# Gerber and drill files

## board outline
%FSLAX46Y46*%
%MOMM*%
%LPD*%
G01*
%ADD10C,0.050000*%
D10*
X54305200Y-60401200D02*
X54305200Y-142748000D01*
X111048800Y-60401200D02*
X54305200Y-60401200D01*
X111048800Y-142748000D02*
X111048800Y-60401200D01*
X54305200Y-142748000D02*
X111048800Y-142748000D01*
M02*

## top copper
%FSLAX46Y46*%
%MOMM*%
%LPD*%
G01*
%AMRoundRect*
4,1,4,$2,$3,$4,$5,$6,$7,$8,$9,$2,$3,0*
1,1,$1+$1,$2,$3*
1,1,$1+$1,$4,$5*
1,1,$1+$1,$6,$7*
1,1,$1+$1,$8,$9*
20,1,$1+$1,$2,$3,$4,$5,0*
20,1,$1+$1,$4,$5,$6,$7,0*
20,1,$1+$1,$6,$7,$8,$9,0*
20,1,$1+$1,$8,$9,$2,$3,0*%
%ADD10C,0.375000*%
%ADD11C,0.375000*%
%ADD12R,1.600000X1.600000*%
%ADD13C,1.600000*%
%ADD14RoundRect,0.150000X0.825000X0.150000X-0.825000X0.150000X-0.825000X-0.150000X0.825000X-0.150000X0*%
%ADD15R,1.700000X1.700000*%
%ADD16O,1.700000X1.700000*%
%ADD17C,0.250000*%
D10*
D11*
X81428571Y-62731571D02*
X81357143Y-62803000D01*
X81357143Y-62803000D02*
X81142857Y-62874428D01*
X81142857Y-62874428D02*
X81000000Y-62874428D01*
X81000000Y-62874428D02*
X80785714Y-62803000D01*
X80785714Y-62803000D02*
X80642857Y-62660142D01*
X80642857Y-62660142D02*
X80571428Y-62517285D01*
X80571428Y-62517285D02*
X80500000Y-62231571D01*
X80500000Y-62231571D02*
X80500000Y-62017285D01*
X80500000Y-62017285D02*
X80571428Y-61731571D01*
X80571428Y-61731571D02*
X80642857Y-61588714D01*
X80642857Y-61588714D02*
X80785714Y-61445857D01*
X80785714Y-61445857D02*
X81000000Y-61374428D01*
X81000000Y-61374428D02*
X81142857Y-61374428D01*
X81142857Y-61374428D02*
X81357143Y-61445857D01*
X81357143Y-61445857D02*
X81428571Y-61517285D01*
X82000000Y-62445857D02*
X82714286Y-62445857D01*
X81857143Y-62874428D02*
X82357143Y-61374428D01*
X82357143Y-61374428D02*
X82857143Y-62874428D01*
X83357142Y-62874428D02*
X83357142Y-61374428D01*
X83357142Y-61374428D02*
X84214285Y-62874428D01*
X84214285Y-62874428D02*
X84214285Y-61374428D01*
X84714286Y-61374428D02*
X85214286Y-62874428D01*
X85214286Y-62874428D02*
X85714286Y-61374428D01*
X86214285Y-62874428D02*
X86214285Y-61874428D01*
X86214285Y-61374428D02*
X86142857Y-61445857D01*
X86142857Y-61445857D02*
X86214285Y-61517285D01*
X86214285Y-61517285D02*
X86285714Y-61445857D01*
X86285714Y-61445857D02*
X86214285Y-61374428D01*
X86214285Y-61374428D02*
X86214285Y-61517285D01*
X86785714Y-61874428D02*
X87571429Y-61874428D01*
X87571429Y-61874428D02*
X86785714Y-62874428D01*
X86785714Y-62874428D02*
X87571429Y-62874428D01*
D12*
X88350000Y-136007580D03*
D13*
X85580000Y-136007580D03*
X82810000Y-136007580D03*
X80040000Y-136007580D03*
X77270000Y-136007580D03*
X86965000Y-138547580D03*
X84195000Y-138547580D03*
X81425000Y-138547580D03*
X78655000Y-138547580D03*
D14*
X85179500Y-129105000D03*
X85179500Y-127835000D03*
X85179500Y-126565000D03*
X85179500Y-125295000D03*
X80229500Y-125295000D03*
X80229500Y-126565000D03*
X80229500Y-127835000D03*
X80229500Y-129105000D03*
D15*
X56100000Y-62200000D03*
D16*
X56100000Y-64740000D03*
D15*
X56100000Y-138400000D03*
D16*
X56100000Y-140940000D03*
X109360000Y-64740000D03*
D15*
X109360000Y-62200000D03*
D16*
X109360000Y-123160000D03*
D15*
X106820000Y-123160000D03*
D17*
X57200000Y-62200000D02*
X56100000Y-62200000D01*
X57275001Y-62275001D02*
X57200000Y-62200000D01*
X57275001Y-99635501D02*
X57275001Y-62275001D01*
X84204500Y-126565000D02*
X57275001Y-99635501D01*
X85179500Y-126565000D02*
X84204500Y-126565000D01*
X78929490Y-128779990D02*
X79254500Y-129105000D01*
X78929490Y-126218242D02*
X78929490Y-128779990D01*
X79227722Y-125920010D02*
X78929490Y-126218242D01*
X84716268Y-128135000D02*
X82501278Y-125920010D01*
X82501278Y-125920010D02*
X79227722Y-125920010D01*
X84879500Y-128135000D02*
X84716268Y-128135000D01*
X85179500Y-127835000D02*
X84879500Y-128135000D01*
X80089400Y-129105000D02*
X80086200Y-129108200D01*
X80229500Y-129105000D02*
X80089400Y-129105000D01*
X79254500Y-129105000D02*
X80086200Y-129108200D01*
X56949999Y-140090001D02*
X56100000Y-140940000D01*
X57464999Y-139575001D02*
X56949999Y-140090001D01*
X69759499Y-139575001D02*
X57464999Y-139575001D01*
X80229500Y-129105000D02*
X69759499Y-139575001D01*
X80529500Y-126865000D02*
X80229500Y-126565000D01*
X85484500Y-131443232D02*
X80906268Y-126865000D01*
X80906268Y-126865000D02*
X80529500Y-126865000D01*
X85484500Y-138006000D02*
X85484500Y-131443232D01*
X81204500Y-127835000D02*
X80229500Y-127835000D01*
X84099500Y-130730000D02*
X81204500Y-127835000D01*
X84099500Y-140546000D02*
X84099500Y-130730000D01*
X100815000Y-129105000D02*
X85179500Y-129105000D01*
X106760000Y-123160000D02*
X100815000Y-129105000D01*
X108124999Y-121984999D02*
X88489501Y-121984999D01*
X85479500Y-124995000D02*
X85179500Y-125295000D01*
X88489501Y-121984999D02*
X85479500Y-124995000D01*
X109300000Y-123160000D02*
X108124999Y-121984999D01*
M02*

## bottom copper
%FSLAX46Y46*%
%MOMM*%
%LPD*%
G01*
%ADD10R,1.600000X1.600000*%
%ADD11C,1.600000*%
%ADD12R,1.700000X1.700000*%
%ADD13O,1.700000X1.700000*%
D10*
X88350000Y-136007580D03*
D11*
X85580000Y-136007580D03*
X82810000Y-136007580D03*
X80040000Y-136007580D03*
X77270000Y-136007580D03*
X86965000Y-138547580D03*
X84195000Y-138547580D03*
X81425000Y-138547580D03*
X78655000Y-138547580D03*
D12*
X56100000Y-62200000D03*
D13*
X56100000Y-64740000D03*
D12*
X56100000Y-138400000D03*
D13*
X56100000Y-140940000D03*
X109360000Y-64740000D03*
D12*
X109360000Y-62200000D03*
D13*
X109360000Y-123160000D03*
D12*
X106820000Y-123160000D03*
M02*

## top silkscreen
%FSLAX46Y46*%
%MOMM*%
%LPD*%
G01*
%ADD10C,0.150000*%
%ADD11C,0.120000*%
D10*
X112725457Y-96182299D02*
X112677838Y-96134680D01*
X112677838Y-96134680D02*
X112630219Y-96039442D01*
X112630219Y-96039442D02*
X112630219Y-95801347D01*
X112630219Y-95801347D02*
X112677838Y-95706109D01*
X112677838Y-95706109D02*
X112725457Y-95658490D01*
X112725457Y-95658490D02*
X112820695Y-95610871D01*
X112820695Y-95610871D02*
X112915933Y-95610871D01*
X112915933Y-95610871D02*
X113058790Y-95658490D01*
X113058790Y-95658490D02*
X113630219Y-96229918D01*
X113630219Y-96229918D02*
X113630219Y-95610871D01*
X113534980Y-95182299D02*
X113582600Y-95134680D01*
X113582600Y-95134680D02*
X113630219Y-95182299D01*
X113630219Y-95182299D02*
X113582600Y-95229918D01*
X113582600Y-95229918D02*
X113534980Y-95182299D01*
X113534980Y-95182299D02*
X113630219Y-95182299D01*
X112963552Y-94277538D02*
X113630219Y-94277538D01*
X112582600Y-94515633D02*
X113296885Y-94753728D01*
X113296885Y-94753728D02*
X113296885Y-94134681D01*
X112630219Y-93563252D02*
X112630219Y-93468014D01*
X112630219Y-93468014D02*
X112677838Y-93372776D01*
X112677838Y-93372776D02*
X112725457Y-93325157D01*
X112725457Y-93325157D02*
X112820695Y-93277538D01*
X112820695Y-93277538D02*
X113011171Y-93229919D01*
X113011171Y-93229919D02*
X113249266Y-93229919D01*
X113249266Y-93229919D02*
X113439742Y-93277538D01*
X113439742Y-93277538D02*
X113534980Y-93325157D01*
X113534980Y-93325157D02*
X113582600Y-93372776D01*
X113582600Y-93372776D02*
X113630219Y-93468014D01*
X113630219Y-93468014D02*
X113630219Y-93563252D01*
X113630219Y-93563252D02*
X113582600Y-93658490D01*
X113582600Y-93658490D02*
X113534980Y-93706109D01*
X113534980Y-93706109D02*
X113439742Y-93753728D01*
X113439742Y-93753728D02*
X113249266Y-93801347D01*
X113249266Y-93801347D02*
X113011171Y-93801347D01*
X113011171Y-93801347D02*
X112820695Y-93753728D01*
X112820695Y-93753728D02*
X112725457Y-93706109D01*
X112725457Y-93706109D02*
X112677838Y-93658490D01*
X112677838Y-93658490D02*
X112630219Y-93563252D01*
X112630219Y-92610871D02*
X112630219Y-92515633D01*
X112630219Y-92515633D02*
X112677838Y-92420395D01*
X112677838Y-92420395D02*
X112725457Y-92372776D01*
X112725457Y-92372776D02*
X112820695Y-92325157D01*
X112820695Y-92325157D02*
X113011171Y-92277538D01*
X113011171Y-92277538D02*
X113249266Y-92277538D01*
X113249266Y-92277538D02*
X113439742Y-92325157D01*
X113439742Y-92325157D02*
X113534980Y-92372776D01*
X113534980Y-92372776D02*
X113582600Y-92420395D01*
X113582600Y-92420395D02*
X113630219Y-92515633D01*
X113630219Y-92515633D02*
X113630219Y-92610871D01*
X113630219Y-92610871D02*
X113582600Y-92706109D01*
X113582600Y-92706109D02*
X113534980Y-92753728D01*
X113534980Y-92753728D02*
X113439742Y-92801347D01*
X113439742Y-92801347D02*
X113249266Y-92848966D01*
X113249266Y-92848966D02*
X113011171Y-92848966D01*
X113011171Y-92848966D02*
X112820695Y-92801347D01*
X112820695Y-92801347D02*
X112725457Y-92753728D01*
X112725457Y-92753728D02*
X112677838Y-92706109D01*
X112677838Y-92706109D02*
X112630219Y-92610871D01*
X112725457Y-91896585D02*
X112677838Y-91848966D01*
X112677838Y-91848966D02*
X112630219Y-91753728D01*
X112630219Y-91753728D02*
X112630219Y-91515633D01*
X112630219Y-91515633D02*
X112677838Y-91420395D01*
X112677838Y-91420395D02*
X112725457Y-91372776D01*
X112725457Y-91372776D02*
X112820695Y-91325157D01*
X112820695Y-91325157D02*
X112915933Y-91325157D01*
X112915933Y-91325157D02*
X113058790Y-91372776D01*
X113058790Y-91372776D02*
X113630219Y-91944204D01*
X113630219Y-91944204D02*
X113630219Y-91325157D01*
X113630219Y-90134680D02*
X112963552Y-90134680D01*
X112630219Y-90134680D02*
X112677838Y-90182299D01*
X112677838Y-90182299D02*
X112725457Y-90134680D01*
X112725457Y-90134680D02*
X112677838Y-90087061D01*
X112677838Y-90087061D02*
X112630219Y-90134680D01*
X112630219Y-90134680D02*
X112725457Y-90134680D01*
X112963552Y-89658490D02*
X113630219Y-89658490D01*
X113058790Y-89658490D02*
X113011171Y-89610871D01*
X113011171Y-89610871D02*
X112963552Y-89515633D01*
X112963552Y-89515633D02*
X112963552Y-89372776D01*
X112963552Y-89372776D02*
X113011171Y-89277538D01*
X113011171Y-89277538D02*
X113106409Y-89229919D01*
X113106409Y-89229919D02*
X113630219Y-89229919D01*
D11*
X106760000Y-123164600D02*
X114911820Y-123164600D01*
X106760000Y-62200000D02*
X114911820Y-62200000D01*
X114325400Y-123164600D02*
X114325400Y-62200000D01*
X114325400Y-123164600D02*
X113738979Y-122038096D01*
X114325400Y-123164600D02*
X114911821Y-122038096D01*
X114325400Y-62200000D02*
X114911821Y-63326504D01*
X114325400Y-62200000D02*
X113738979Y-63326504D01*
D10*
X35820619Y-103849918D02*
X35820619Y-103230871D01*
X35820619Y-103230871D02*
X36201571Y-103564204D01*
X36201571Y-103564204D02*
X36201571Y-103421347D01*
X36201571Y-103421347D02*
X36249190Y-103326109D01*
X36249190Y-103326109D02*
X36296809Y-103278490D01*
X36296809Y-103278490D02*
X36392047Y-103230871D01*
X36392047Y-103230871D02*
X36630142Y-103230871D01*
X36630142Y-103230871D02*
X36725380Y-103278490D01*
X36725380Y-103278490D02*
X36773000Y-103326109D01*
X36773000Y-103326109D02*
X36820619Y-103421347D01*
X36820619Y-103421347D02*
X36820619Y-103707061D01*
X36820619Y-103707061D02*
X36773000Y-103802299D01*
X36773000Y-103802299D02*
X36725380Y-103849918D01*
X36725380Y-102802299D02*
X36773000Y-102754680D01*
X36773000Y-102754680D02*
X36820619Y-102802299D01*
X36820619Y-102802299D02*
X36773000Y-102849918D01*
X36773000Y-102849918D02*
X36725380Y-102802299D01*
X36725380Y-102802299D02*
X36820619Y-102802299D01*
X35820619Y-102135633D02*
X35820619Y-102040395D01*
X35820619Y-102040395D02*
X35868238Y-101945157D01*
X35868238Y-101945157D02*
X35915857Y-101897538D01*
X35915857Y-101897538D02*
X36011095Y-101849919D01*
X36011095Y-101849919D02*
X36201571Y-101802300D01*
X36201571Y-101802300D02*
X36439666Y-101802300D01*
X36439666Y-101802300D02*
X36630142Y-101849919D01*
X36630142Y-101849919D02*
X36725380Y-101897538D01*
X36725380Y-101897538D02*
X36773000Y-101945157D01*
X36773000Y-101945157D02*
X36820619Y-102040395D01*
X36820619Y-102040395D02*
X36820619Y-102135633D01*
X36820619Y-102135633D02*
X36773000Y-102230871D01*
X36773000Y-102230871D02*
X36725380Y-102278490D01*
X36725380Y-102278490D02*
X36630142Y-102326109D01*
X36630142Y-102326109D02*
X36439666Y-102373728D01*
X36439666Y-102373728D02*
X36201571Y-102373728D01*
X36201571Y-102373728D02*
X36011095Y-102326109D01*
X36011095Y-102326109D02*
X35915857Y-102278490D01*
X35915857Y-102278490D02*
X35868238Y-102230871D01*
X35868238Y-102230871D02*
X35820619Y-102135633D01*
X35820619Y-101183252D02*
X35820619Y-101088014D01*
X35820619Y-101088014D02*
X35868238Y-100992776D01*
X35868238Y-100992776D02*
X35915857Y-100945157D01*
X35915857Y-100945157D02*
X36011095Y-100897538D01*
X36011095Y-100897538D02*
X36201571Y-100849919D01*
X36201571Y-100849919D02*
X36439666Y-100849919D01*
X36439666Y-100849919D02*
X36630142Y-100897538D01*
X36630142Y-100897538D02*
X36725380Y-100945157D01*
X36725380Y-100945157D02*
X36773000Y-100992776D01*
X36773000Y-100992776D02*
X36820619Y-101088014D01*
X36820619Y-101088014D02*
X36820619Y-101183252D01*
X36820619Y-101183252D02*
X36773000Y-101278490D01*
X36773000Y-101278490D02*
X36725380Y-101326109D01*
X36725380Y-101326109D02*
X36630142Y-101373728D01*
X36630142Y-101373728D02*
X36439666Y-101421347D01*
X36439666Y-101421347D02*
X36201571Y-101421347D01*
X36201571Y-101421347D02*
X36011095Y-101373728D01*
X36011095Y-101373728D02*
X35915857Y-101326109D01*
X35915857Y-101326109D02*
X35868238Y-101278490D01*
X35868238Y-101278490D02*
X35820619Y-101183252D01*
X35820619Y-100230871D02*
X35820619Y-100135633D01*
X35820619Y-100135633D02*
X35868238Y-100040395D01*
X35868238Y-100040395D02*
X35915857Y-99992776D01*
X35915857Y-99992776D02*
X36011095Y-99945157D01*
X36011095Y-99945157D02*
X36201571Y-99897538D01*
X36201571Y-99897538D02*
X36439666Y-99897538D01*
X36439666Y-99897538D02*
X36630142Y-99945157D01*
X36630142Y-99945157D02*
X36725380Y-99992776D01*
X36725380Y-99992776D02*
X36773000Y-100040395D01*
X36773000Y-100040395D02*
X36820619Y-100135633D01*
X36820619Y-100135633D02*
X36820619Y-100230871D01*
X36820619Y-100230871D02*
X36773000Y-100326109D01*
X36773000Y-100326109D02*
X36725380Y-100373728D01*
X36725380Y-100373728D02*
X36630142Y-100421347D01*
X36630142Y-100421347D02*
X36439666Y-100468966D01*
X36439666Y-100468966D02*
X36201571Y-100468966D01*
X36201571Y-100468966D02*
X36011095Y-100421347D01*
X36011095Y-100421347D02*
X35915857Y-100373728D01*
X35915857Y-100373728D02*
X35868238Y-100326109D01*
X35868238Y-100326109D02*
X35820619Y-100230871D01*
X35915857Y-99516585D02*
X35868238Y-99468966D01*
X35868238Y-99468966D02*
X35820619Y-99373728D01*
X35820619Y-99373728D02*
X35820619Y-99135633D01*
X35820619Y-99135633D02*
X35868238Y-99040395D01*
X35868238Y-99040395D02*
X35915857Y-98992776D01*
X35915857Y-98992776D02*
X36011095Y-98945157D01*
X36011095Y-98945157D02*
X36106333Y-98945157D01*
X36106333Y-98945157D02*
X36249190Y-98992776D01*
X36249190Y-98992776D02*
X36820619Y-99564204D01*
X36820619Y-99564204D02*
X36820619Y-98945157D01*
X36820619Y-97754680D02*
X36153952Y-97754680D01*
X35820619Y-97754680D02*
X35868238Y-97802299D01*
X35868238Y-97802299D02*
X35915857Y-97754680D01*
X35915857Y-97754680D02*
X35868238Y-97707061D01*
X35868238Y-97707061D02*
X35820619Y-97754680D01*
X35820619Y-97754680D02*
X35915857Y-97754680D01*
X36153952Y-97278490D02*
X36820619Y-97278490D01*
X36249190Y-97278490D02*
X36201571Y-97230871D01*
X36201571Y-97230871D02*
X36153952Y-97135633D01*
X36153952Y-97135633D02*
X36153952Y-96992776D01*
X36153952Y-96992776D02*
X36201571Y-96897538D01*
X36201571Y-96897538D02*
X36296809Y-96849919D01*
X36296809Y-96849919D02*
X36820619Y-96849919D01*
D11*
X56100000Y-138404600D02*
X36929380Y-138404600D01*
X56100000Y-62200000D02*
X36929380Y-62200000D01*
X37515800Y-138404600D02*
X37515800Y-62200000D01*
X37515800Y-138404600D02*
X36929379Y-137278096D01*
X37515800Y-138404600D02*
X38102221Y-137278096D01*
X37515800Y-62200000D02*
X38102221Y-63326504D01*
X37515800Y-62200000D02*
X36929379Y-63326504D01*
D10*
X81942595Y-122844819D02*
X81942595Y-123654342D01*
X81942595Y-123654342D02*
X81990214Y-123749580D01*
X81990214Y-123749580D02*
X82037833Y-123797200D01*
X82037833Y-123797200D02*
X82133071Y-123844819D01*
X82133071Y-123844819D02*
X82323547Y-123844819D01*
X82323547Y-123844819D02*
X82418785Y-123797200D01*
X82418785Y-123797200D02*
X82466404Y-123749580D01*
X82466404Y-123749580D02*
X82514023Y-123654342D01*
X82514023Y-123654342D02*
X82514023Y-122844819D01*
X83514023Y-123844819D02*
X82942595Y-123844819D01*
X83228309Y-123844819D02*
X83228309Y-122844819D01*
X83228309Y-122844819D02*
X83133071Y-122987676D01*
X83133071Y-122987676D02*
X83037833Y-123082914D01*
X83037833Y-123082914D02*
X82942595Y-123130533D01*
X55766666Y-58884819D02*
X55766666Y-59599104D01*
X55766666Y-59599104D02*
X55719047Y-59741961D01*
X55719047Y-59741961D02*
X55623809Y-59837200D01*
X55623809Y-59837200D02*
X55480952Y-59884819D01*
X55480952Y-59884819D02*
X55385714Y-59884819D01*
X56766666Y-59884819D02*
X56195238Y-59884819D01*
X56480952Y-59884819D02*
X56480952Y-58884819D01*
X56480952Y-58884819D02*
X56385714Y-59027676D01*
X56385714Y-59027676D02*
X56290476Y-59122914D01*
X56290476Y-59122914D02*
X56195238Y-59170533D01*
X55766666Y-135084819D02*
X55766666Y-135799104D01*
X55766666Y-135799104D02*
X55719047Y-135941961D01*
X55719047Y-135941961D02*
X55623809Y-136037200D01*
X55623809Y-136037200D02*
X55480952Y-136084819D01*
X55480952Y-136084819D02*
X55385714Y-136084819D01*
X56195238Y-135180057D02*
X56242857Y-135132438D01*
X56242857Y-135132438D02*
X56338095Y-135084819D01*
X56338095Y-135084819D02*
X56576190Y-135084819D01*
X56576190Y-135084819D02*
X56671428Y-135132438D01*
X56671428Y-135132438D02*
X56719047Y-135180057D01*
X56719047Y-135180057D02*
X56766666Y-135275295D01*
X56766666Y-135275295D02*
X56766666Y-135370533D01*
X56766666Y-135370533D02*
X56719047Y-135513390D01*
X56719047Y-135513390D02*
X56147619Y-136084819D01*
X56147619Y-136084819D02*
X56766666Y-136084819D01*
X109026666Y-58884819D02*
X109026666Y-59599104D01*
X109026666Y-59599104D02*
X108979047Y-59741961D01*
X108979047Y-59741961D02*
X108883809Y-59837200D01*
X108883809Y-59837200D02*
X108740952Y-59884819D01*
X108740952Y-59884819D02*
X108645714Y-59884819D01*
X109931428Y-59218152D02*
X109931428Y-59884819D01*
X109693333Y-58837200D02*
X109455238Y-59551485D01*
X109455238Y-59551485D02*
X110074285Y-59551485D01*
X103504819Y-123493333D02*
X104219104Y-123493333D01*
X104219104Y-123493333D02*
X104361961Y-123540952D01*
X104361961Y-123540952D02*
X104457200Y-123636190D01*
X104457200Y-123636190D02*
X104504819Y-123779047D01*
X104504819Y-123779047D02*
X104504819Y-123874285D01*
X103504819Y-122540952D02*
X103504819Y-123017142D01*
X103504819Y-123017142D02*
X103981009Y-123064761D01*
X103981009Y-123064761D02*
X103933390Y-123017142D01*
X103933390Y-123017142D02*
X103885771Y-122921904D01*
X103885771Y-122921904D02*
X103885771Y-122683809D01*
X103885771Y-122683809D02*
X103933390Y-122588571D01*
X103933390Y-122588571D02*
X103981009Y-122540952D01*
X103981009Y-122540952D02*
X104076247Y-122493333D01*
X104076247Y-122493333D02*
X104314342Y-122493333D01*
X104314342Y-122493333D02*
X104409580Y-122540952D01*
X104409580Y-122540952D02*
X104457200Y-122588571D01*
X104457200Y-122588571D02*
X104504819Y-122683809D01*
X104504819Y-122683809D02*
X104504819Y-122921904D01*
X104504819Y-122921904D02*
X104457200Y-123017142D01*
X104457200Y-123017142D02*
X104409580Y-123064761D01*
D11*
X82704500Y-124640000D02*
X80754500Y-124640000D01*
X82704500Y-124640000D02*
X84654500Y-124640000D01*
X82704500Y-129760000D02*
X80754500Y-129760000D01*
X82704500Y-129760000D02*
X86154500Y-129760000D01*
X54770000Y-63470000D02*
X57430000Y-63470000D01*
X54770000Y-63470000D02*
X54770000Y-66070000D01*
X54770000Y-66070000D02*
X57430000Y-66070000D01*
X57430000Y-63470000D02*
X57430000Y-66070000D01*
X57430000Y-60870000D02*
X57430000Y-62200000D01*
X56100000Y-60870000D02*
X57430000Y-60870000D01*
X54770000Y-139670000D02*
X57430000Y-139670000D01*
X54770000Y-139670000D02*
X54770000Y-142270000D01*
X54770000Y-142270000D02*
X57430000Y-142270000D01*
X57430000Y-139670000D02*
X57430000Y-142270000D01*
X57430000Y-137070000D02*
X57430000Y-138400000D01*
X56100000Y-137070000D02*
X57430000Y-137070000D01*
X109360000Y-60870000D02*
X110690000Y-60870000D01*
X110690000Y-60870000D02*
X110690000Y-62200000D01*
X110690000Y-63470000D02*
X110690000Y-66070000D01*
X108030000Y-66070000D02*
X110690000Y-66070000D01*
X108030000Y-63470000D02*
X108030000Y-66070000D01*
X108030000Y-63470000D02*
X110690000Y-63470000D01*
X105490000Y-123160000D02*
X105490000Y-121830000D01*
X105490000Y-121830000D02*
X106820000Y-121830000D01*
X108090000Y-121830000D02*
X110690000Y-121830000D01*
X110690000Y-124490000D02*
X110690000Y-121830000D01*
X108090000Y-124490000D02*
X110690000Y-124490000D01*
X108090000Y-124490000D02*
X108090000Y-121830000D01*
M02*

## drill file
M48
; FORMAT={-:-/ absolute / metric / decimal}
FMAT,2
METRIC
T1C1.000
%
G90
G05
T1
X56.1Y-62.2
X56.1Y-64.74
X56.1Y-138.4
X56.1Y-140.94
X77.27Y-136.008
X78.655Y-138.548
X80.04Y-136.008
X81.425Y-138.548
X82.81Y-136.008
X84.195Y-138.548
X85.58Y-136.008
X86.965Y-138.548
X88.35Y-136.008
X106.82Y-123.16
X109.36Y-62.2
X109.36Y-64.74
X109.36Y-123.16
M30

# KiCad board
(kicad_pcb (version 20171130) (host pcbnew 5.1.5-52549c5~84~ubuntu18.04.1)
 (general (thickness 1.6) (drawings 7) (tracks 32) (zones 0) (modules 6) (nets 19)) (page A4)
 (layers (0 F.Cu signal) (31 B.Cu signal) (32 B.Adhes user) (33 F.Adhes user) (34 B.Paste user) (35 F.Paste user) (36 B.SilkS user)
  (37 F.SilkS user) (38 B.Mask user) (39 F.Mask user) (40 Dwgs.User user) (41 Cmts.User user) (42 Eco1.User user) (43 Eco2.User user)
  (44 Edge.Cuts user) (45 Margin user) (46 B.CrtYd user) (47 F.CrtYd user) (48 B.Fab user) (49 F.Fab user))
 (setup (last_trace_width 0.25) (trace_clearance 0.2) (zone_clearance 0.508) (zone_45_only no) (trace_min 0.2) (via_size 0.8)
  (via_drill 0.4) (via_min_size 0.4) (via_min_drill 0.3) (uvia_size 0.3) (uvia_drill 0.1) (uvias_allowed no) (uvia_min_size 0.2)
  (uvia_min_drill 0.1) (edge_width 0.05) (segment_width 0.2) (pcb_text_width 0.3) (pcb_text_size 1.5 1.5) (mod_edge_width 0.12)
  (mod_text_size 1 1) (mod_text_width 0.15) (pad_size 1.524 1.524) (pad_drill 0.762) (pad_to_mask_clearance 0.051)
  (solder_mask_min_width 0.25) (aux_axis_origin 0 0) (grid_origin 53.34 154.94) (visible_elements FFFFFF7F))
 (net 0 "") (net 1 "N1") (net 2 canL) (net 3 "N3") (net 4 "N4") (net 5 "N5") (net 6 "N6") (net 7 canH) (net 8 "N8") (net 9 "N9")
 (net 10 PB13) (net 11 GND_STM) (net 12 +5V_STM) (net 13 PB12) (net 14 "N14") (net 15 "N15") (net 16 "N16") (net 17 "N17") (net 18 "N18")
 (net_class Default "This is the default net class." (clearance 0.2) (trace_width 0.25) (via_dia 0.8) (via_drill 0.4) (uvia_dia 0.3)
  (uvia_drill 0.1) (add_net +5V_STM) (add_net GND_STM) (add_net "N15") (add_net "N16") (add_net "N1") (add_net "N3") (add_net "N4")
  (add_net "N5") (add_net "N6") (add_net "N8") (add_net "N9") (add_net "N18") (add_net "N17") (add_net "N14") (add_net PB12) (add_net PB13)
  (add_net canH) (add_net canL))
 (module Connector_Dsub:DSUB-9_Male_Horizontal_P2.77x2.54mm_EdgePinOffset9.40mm (layer B.Cu) (at 88.35 136.00758 180)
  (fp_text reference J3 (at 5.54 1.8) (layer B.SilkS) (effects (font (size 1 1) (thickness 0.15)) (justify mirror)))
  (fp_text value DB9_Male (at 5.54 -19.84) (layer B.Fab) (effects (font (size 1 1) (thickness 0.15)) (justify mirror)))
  (pad 1 thru_hole rect (at 0 0 180) (size 1.6 1.6) (drill 1) (layers *.Cu *.Mask) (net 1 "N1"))
  (pad 2 thru_hole circle (at 2.77 0 180) (size 1.6 1.6) (drill 1) (layers *.Cu *.Mask) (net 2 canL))
  (pad 3 thru_hole circle (at 5.54 0 180) (size 1.6 1.6) (drill 1) (layers *.Cu *.Mask) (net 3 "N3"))
  (pad 4 thru_hole circle (at 8.31 0 180) (size 1.6 1.6) (drill 1) (layers *.Cu *.Mask) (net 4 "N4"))
  (pad 5 thru_hole circle (at 11.08 0 180) (size 1.6 1.6) (drill 1) (layers *.Cu *.Mask) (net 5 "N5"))
  (pad 6 thru_hole circle (at 1.385 -2.54 180) (size 1.6 1.6) (drill 1) (layers *.Cu *.Mask) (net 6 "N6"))
  (pad 7 thru_hole circle (at 4.155 -2.54 180) (size 1.6 1.6) (drill 1) (layers *.Cu *.Mask) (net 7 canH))
  (pad 8 thru_hole circle (at 6.925 -2.54 180) (size 1.6 1.6) (drill 1) (layers *.Cu *.Mask) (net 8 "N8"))
  (pad 9 thru_hole circle (at 9.695 -2.54 180) (size 1.6 1.6) (drill 1) (layers *.Cu *.Mask) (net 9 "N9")))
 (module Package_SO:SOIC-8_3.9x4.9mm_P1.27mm (layer F.Cu) (at 82.7045 127.2 180)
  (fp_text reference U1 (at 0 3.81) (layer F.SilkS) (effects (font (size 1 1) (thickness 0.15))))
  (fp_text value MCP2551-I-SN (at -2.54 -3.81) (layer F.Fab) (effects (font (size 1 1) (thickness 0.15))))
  (fp_line (start 0 2.56) (end 1.95 2.56) (layer F.SilkS) (width 0.12))
  (fp_line (start 0 2.56) (end -1.95 2.56) (layer F.SilkS) (width 0.12))
  (fp_line (start 0 -2.56) (end 1.95 -2.56) (layer F.SilkS) (width 0.12))
  (fp_line (start 0 -2.56) (end -3.45 -2.56) (layer F.SilkS) (width 0.12))
  (pad 1 smd roundrect (at -2.475 -1.905 180) (size 1.95 0.6) (layers F.Cu F.Paste F.Mask) (roundrect_rratio 0.25) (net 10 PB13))
  (pad 2 smd roundrect (at -2.475 -0.635 180) (size 1.95 0.6) (layers F.Cu F.Paste F.Mask) (roundrect_rratio 0.25) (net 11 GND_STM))
  (pad 3 smd roundrect (at -2.475 0.635 180) (size 1.95 0.6) (layers F.Cu F.Paste F.Mask) (roundrect_rratio 0.25) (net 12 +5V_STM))
  (pad 4 smd roundrect (at -2.475 1.905 180) (size 1.95 0.6) (layers F.Cu F.Paste F.Mask) (roundrect_rratio 0.25) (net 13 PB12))
  (pad 5 smd roundrect (at 2.475 1.905 180) (size 1.95 0.6) (layers F.Cu F.Paste F.Mask) (roundrect_rratio 0.25) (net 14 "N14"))
  (pad 6 smd roundrect (at 2.475 0.635 180) (size 1.95 0.6) (layers F.Cu F.Paste F.Mask) (roundrect_rratio 0.25) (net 2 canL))
  (pad 7 smd roundrect (at 2.475 -0.635 180) (size 1.95 0.6) (layers F.Cu F.Paste F.Mask) (roundrect_rratio 0.25) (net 7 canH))
  (pad 8 smd roundrect (at 2.475 -1.905 180) (size 1.95 0.6) (layers F.Cu F.Paste F.Mask) (roundrect_rratio 0.25) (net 11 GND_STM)))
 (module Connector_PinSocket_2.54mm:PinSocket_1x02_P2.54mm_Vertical (layer F.Cu) (at 56.1 62.2)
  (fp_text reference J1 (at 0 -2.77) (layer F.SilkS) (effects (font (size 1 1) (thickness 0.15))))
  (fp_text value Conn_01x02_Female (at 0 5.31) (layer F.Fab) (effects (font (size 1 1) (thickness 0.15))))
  (fp_line (start -1.33 1.27) (end 1.33 1.27) (layer F.SilkS) (width 0.12))
  (fp_line (start -1.33 1.27) (end -1.33 3.87) (layer F.SilkS) (width 0.12))
  (fp_line (start -1.33 3.87) (end 1.33 3.87) (layer F.SilkS) (width 0.12))
  (fp_line (start 1.33 1.27) (end 1.33 3.87) (layer F.SilkS) (width 0.12))
  (fp_line (start 1.33 -1.33) (end 1.33 0) (layer F.SilkS) (width 0.12))
  (fp_line (start 0 -1.33) (end 1.33 -1.33) (layer F.SilkS) (width 0.12))
  (pad 1 thru_hole rect (at 0 0) (size 1.7 1.7) (drill 1) (layers *.Cu *.Mask) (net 12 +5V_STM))
  (pad 2 thru_hole oval (at 0 2.54) (size 1.7 1.7) (drill 1) (layers *.Cu *.Mask) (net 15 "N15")))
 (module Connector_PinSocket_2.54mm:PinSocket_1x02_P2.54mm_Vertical (layer F.Cu) (at 56.1 138.4)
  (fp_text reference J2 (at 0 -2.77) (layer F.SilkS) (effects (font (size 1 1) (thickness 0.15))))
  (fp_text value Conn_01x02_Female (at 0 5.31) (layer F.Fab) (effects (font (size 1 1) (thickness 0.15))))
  (fp_line (start -1.33 1.27) (end 1.33 1.27) (layer F.SilkS) (width 0.12))
  (fp_line (start -1.33 1.27) (end -1.33 3.87) (layer F.SilkS) (width 0.12))
  (fp_line (start -1.33 3.87) (end 1.33 3.87) (layer F.SilkS) (width 0.12))
  (fp_line (start 1.33 1.27) (end 1.33 3.87) (layer F.SilkS) (width 0.12))
  (fp_line (start 1.33 -1.33) (end 1.33 0) (layer F.SilkS) (width 0.12))
  (fp_line (start 0 -1.33) (end 1.33 -1.33) (layer F.SilkS) (width 0.12))
  (pad 1 thru_hole rect (at 0 0) (size 1.7 1.7) (drill 1) (layers *.Cu *.Mask) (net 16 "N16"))
  (pad 2 thru_hole oval (at 0 2.54) (size 1.7 1.7) (drill 1) (layers *.Cu *.Mask) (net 11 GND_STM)))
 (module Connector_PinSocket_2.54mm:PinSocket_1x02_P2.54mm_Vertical (layer F.Cu) (at 109.36 62.2)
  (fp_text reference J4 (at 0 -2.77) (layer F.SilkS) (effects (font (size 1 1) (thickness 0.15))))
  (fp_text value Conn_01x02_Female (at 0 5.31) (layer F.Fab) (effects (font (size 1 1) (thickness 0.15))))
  (fp_line (start 0 -1.33) (end 1.33 -1.33) (layer F.SilkS) (width 0.12))
  (fp_line (start 1.33 -1.33) (end 1.33 0) (layer F.SilkS) (width 0.12))
  (fp_line (start 1.33 1.27) (end 1.33 3.87) (layer F.SilkS) (width 0.12))
  (fp_line (start -1.33 3.87) (end 1.33 3.87) (layer F.SilkS) (width 0.12))
  (fp_line (start -1.33 1.27) (end -1.33 3.87) (layer F.SilkS) (width 0.12))
  (fp_line (start -1.33 1.27) (end 1.33 1.27) (layer F.SilkS) (width 0.12))
  (pad 2 thru_hole oval (at 0 2.54) (size 1.7 1.7) (drill 1) (layers *.Cu *.Mask) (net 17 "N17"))
  (pad 1 thru_hole rect (at 0 0) (size 1.7 1.7) (drill 1) (layers *.Cu *.Mask) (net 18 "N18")))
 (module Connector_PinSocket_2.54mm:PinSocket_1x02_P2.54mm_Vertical (layer F.Cu) (at 106.82 123.16 90)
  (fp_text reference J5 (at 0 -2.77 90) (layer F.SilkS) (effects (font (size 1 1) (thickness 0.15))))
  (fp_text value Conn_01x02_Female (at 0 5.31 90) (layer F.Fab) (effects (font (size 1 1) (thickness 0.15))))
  (fp_line (start 0 -1.33) (end 1.33 -1.33) (layer F.SilkS) (width 0.12))
  (fp_line (start 1.33 -1.33) (end 1.33 0) (layer F.SilkS) (width 0.12))
  (fp_line (start 1.33 1.27) (end 1.33 3.87) (layer F.SilkS) (width 0.12))
  (fp_line (start -1.33 3.87) (end 1.33 3.87) (layer F.SilkS) (width 0.12))
  (fp_line (start -1.33 1.27) (end -1.33 3.87) (layer F.SilkS) (width 0.12))
  (fp_line (start -1.33 1.27) (end 1.33 1.27) (layer F.SilkS) (width 0.12))
  (pad 2 thru_hole oval (at 0 2.54 90) (size 1.7 1.7) (drill 1) (layers *.Cu *.Mask) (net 13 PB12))
  (pad 1 thru_hole rect (at 0 0 90) (size 1.7 1.7) (drill 1) (layers *.Cu *.Mask) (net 10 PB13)))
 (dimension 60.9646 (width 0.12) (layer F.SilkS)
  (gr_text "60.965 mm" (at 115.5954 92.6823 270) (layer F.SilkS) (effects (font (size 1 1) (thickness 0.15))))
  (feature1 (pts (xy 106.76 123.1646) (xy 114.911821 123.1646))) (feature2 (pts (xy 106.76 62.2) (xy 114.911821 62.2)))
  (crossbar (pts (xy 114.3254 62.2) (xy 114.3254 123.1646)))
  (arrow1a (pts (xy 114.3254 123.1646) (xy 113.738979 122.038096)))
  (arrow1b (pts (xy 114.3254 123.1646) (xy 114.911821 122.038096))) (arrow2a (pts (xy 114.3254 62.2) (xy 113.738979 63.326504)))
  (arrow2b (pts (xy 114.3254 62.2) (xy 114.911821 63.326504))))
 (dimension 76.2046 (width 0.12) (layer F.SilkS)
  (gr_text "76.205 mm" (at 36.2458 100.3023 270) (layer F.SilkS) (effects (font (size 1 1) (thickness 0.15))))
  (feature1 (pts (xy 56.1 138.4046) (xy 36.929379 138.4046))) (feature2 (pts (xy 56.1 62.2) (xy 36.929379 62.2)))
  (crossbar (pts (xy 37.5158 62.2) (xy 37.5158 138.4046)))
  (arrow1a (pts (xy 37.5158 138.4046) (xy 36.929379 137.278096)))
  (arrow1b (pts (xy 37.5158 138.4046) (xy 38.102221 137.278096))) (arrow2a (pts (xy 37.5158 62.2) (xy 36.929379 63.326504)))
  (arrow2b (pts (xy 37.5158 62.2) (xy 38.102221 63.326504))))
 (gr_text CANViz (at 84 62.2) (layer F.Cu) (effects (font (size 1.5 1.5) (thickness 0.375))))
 (gr_line (start 54.3052 60.4012) (end 54.3052 142.748) (layer Edge.Cuts) (width 0.05))
 (gr_line (start 111.0488 60.4012) (end 54.3052 60.4012) (layer Edge.Cuts) (width 0.05))
 (gr_line (start 111.0488 142.748) (end 111.0488 60.4012) (layer Edge.Cuts) (width 0.05))
 (gr_line (start 54.3052 142.748) (end 111.0488 142.748) (layer Edge.Cuts) (width 0.05))
 (segment (start 57.2 62.2) (end 56.1 62.2) (width 0.25) (layer F.Cu) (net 12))
 (segment (start 57.275001 62.275001) (end 57.2 62.2) (width 0.25) (layer F.Cu) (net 12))
 (segment (start 57.275001 99.635501) (end 57.275001 62.275001) (width 0.25) (layer F.Cu) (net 12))
 (segment (start 84.2045 126.565) (end 57.275001 99.635501) (width 0.25) (layer F.Cu) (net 12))
 (segment (start 85.1795 126.565) (end 84.2045 126.565) (width 0.25) (layer F.Cu) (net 12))
 (segment (start 78.92949 128.77999) (end 79.2545 129.105) (width 0.25) (layer F.Cu) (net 11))
 (segment (start 78.92949 126.218242) (end 78.92949 128.77999) (width 0.25) (layer F.Cu) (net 11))
 (segment (start 79.227722 125.92001) (end 78.92949 126.218242) (width 0.25) (layer F.Cu) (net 11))
 (segment (start 84.716268 128.135) (end 82.501278 125.92001) (width 0.25) (layer F.Cu) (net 11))
 (segment (start 82.501278 125.92001) (end 79.227722 125.92001) (width 0.25) (layer F.Cu) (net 11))
 (segment (start 84.8795 128.135) (end 84.716268 128.135) (width 0.25) (layer F.Cu) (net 11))
 (segment (start 85.1795 127.835) (end 84.8795 128.135) (width 0.25) (layer F.Cu) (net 11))
 (segment (start 80.0894 129.105) (end 80.0862 129.1082) (width 0.25) (layer F.Cu) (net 11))
 (segment (start 80.2295 129.105) (end 80.0894 129.105) (width 0.25) (layer F.Cu) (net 11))
 (segment (start 79.2545 129.105) (end 80.0862 129.1082) (width 0.25) (layer F.Cu) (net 11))
 (segment (start 56.949999 140.090001) (end 56.1 140.94) (width 0.25) (layer F.Cu) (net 11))
 (segment (start 57.464999 139.575001) (end 56.949999 140.090001) (width 0.25) (layer F.Cu) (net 11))
 (segment (start 69.759499 139.575001) (end 57.464999 139.575001) (width 0.25) (layer F.Cu) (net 11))
 (segment (start 80.2295 129.105) (end 69.759499 139.575001) (width 0.25) (layer F.Cu) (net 11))
 (segment (start 80.5295 126.865) (end 80.2295 126.565) (width 0.25) (layer F.Cu) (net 2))
 (segment (start 85.4845 131.443232) (end 80.906268 126.865) (width 0.25) (layer F.Cu) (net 2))
 (segment (start 80.906268 126.865) (end 80.5295 126.865) (width 0.25) (layer F.Cu) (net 2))
 (segment (start 85.4845 138.006) (end 85.4845 131.443232) (width 0.25) (layer F.Cu) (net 2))
 (segment (start 81.2045 127.835) (end 80.2295 127.835) (width 0.25) (layer F.Cu) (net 7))
 (segment (start 84.0995 130.73) (end 81.2045 127.835) (width 0.25) (layer F.Cu) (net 7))
 (segment (start 84.0995 140.546) (end 84.0995 130.73) (width 0.25) (layer F.Cu) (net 7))
 (segment (start 100.815 129.105) (end 85.1795 129.105) (width 0.25) (layer F.Cu) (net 10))
 (segment (start 106.76 123.16) (end 100.815 129.105) (width 0.25) (layer F.Cu) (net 10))
 (segment (start 108.124999 121.984999) (end 88.489501 121.984999) (width 0.25) (layer F.Cu) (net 13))
 (segment (start 85.4795 124.995) (end 85.1795 125.295) (width 0.25) (layer F.Cu) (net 13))
 (segment (start 88.489501 121.984999) (end 85.4795 124.995) (width 0.25) (layer F.Cu) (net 13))
 (segment (start 109.3 123.16) (end 108.124999 121.984999) (width 0.25) (layer F.Cu) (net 13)))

